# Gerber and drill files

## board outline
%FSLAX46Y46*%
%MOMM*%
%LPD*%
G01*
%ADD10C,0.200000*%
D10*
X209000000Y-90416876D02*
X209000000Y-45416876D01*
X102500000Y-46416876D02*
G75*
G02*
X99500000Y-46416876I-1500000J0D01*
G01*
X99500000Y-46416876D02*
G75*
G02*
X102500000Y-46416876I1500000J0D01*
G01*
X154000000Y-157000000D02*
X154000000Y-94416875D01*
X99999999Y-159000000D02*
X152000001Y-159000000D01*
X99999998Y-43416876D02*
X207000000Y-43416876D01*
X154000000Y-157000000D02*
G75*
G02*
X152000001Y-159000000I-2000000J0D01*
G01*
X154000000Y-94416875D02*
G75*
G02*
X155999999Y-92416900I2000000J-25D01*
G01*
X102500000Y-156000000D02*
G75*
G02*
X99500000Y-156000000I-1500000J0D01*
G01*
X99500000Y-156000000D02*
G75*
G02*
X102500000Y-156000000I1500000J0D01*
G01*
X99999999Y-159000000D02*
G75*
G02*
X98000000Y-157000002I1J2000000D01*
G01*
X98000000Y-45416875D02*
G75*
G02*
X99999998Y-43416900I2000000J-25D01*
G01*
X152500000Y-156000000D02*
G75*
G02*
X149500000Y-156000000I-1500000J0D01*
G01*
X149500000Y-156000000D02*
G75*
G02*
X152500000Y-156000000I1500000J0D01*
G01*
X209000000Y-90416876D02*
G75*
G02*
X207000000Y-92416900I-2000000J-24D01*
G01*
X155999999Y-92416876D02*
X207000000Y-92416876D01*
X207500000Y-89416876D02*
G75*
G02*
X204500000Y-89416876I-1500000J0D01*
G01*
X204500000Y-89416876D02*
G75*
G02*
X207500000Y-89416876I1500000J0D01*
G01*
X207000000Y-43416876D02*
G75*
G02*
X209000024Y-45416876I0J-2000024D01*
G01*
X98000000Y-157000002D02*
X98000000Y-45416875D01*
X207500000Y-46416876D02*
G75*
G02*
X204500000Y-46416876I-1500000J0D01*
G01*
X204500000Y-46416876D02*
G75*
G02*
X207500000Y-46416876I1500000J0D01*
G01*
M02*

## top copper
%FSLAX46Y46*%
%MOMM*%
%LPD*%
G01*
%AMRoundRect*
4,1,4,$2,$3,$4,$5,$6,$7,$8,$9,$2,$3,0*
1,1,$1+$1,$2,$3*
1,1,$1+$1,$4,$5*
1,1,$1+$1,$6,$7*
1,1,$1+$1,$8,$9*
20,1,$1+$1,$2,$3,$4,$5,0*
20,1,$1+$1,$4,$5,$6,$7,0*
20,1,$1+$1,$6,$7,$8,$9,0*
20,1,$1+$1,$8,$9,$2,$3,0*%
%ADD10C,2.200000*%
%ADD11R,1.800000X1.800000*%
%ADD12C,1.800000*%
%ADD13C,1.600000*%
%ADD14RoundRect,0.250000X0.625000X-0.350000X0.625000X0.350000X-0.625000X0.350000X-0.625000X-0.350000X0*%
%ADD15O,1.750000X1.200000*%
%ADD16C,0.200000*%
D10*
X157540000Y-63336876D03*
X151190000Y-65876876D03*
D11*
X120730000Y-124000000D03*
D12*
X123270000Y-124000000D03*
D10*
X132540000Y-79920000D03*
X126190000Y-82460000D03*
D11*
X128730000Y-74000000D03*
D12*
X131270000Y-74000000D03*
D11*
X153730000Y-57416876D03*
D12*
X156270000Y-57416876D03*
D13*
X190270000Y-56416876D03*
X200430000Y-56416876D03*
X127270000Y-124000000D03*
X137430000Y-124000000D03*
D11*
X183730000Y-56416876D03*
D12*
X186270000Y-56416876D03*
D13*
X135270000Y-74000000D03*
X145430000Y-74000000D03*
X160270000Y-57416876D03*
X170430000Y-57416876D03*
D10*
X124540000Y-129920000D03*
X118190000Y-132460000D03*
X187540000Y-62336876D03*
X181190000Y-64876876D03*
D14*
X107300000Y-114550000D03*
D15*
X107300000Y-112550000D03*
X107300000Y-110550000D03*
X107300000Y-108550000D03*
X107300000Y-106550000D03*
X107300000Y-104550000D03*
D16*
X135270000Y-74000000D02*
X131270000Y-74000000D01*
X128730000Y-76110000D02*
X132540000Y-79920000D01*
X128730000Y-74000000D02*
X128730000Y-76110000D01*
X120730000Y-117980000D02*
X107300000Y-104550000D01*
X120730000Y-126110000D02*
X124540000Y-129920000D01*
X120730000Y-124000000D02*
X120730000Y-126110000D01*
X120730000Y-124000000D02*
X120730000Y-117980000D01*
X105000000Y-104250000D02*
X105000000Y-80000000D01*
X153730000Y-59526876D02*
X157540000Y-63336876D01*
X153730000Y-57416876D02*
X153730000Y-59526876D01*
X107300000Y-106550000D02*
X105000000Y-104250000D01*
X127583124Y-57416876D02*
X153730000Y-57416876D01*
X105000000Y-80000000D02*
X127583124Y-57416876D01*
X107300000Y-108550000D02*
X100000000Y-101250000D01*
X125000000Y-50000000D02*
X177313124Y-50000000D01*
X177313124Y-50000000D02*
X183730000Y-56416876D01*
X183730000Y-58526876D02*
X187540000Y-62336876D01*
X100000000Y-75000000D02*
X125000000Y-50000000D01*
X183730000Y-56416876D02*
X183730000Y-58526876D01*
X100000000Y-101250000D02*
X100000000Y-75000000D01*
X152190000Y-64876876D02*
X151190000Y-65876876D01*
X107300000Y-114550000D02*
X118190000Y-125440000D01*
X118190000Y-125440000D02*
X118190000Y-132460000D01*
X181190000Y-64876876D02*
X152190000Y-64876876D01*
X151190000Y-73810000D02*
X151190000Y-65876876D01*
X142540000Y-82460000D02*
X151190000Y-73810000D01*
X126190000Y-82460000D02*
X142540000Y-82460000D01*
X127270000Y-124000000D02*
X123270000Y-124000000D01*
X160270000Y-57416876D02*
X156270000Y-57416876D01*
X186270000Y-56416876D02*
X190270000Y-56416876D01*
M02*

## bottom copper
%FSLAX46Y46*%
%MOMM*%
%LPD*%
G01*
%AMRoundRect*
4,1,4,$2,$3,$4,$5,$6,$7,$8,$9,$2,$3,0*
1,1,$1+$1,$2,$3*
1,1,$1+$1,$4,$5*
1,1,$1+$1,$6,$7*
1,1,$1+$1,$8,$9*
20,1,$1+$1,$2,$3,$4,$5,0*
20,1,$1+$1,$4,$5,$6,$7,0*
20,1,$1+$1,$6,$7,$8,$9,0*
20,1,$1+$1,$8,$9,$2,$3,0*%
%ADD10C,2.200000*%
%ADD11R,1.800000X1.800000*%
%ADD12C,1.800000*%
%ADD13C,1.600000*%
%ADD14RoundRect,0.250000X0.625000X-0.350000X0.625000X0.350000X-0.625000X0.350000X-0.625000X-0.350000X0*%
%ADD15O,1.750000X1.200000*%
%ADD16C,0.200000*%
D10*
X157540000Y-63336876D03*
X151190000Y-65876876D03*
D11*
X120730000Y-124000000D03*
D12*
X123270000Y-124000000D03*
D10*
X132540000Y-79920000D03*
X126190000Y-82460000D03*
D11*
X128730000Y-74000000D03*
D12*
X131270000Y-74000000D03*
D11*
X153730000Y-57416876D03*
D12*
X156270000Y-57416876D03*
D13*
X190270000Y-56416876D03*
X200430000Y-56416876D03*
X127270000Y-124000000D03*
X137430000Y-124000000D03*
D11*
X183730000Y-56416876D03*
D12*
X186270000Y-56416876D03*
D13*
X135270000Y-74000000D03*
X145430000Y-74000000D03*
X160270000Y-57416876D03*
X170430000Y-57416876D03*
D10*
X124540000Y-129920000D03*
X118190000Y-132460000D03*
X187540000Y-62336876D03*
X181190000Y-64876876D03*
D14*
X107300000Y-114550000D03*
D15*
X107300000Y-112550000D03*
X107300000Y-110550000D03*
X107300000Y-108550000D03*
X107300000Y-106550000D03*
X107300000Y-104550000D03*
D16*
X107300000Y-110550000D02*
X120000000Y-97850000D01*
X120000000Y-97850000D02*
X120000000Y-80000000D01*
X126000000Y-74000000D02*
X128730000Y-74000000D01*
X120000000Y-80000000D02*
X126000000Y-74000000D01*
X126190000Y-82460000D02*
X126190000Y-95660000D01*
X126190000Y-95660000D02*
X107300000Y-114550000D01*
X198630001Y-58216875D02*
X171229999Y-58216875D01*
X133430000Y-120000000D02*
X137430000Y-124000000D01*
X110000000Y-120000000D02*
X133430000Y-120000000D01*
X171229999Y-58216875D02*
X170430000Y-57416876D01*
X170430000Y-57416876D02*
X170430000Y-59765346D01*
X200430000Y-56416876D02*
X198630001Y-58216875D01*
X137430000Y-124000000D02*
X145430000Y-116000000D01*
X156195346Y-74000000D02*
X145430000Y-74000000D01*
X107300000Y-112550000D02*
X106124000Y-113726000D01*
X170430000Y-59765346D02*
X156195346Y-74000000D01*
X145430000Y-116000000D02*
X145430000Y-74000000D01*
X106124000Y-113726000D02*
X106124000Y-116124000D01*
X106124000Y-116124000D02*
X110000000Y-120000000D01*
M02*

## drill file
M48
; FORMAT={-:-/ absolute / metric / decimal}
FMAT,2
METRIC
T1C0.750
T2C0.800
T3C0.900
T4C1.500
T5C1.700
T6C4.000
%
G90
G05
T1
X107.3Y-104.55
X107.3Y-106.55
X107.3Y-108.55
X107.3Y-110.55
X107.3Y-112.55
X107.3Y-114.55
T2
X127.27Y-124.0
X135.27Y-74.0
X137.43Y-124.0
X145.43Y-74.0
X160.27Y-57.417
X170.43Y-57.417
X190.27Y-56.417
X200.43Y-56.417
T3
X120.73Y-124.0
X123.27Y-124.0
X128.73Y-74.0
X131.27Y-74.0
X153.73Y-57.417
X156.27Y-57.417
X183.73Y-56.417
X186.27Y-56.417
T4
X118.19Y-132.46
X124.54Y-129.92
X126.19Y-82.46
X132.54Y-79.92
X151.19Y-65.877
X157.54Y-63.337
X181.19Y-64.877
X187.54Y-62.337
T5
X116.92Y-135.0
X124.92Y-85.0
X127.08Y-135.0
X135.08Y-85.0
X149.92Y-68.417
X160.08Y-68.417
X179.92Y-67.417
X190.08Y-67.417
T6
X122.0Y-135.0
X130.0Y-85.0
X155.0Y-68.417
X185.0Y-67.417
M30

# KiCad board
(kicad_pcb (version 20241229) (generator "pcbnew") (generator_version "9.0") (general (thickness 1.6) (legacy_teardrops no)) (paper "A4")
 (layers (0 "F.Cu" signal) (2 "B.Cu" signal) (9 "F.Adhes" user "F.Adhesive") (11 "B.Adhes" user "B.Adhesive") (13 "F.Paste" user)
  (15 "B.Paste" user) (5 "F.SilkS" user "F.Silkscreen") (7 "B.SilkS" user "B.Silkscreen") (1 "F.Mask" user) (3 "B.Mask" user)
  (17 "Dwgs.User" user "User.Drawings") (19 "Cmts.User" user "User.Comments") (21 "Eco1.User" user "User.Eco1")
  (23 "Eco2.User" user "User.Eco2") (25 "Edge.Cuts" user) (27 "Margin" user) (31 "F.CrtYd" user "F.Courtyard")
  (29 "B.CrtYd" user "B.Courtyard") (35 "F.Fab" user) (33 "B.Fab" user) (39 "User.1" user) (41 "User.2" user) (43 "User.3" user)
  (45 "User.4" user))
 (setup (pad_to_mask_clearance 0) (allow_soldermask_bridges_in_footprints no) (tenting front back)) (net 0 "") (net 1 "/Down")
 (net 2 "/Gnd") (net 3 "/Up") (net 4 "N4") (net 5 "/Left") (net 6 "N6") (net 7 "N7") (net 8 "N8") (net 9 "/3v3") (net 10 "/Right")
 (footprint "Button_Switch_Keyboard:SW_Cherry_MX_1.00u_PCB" (layer "F.Cu") (at 157.54 63.336876)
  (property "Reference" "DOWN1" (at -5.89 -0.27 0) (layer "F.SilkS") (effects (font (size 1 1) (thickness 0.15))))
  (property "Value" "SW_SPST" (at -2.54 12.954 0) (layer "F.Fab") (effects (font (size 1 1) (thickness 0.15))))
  (pad "" np_thru_hole circle (at -7.62 5.08) (size 1.7 1.7) (drill 1.7) (layers "*.Cu" "*.Mask"))
  (pad "" np_thru_hole circle (at -2.54 5.08) (size 4 4) (drill 4) (layers "*.Cu" "*.Mask"))
  (pad "" np_thru_hole circle (at 2.54 5.08) (size 1.7 1.7) (drill 1.7) (layers "*.Cu" "*.Mask"))
  (pad "1" thru_hole circle (at 0 0) (size 2.2 2.2) (drill 1.5) (layers "*.Cu" "*.Mask") (remove_unused_layers no) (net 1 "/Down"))
  (pad "2" thru_hole circle (at -6.35 2.54) (size 2.2 2.2) (drill 1.5) (layers "*.Cu" "*.Mask") (remove_unused_layers no) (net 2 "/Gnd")))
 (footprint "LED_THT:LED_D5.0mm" (layer "F.Cu") (at 120.73 124)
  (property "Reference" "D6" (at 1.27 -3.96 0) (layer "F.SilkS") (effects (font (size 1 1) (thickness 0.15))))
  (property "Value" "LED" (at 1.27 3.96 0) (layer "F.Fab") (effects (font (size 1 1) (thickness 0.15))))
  (pad "1" thru_hole rect (at 0 0) (size 1.8 1.8) (drill 0.9) (layers "*.Cu" "*.Mask") (remove_unused_layers no) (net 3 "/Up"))
  (pad "2" thru_hole circle (at 2.54 0) (size 1.8 1.8) (drill 0.9) (layers "*.Cu" "*.Mask") (remove_unused_layers no) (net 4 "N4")))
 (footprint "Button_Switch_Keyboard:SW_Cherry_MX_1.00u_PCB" (layer "F.Cu") (at 132.54 79.92)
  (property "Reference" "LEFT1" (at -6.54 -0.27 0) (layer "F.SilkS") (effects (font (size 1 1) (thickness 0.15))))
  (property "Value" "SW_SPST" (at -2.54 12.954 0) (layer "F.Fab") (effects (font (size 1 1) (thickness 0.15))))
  (pad "" np_thru_hole circle (at -7.62 5.08) (size 1.7 1.7) (drill 1.7) (layers "*.Cu" "*.Mask"))
  (pad "" np_thru_hole circle (at -2.54 5.08) (size 4 4) (drill 4) (layers "*.Cu" "*.Mask"))
  (pad "" np_thru_hole circle (at 2.54 5.08) (size 1.7 1.7) (drill 1.7) (layers "*.Cu" "*.Mask"))
  (pad "1" thru_hole circle (at 0 0) (size 2.2 2.2) (drill 1.5) (layers "*.Cu" "*.Mask") (remove_unused_layers no) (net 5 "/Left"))
  (pad "2" thru_hole circle (at -6.35 2.54) (size 2.2 2.2) (drill 1.5) (layers "*.Cu" "*.Mask") (remove_unused_layers no) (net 2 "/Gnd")))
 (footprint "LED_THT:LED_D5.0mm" (layer "F.Cu") (at 128.73 74)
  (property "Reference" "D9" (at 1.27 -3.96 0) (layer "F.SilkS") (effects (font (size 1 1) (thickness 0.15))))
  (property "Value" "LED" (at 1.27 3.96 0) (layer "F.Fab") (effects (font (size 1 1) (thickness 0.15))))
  (pad "1" thru_hole rect (at 0 0) (size 1.8 1.8) (drill 0.9) (layers "*.Cu" "*.Mask") (remove_unused_layers no) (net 5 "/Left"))
  (pad "2" thru_hole circle (at 2.54 0) (size 1.8 1.8) (drill 0.9) (layers "*.Cu" "*.Mask") (remove_unused_layers no) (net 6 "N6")))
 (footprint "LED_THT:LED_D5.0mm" (layer "F.Cu") (at 153.73 57.416876)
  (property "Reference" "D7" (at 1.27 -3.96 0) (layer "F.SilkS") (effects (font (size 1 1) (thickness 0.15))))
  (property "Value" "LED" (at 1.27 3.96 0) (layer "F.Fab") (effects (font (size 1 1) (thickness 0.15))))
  (pad "1" thru_hole rect (at 0 0) (size 1.8 1.8) (drill 0.9) (layers "*.Cu" "*.Mask") (remove_unused_layers no) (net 1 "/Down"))
  (pad "2" thru_hole circle (at 2.54 0) (size 1.8 1.8) (drill 0.9) (layers "*.Cu" "*.Mask") (remove_unused_layers no) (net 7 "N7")))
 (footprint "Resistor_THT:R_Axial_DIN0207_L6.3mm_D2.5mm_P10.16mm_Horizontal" (layer "F.Cu") (at 190.27 56.416876)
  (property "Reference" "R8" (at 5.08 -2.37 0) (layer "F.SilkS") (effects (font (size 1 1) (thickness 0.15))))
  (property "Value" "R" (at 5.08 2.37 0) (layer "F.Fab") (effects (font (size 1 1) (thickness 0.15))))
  (pad "1" thru_hole circle (at 0 0) (size 1.6 1.6) (drill 0.8) (layers "*.Cu" "*.Mask") (remove_unused_layers no) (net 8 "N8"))
  (pad "2" thru_hole circle (at 10.16 0) (size 1.6 1.6) (drill 0.8) (layers "*.Cu" "*.Mask") (remove_unused_layers no) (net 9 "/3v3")))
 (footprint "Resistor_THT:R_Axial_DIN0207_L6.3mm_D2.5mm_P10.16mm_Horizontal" (layer "F.Cu") (at 127.27 124)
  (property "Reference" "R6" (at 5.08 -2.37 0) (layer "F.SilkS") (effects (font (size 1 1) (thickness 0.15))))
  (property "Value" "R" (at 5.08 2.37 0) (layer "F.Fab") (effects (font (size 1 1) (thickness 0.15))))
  (pad "1" thru_hole circle (at 0 0) (size 1.6 1.6) (drill 0.8) (layers "*.Cu" "*.Mask") (remove_unused_layers no) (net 4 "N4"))
  (pad "2" thru_hole circle (at 10.16 0) (size 1.6 1.6) (drill 0.8) (layers "*.Cu" "*.Mask") (remove_unused_layers no) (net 9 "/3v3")))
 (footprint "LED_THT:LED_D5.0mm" (layer "F.Cu") (at 183.73 56.416876)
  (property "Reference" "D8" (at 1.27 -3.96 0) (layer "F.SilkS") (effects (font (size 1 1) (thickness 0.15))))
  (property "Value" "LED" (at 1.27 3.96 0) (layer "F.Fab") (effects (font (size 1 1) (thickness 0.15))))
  (pad "1" thru_hole rect (at 0 0) (size 1.8 1.8) (drill 0.9) (layers "*.Cu" "*.Mask") (remove_unused_layers no) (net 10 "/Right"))
  (pad "2" thru_hole circle (at 2.54 0) (size 1.8 1.8) (drill 0.9) (layers "*.Cu" "*.Mask") (remove_unused_layers no) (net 8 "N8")))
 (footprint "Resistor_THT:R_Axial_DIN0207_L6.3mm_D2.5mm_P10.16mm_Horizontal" (layer "F.Cu") (at 135.27 74)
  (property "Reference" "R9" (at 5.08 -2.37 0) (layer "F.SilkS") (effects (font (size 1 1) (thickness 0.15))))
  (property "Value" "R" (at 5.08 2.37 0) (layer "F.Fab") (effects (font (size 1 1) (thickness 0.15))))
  (pad "1" thru_hole circle (at 0 0) (size 1.6 1.6) (drill 0.8) (layers "*.Cu" "*.Mask") (remove_unused_layers no) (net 6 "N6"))
  (pad "2" thru_hole circle (at 10.16 0) (size 1.6 1.6) (drill 0.8) (layers "*.Cu" "*.Mask") (remove_unused_layers no) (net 9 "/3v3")))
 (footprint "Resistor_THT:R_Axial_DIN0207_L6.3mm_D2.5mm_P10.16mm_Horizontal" (layer "F.Cu") (at 160.27 57.416876)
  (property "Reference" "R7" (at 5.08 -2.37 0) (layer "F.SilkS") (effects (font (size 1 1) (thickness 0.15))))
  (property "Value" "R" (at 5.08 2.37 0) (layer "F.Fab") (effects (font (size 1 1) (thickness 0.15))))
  (pad "1" thru_hole circle (at 0 0) (size 1.6 1.6) (drill 0.8) (layers "*.Cu" "*.Mask") (remove_unused_layers no) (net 7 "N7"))
  (pad "2" thru_hole circle (at 10.16 0) (size 1.6 1.6) (drill 0.8) (layers "*.Cu" "*.Mask") (remove_unused_layers no) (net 9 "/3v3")))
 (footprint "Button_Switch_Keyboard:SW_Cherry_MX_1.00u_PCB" (layer "F.Cu") (at 124.54 129.92)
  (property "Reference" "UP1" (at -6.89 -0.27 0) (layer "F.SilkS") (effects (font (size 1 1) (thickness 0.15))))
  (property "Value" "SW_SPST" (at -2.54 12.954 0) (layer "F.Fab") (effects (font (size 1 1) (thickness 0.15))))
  (pad "" np_thru_hole circle (at -7.62 5.08) (size 1.7 1.7) (drill 1.7) (layers "*.Cu" "*.Mask"))
  (pad "" np_thru_hole circle (at -2.54 5.08) (size 4 4) (drill 4) (layers "*.Cu" "*.Mask"))
  (pad "" np_thru_hole circle (at 2.54 5.08) (size 1.7 1.7) (drill 1.7) (layers "*.Cu" "*.Mask"))
  (pad "1" thru_hole circle (at 0 0) (size 2.2 2.2) (drill 1.5) (layers "*.Cu" "*.Mask") (remove_unused_layers no) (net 3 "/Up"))
  (pad "2" thru_hole circle (at -6.35 2.54) (size 2.2 2.2) (drill 1.5) (layers "*.Cu" "*.Mask") (remove_unused_layers no) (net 2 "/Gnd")))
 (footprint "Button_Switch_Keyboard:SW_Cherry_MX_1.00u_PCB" (layer "F.Cu") (at 187.54 62.336876)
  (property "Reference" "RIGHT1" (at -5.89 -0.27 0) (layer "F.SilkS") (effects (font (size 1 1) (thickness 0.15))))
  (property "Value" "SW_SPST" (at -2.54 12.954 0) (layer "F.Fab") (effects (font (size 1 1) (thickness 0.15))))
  (pad "" np_thru_hole circle (at -7.62 5.08) (size 1.7 1.7) (drill 1.7) (layers "*.Cu" "*.Mask"))
  (pad "" np_thru_hole circle (at -2.54 5.08) (size 4 4) (drill 4) (layers "*.Cu" "*.Mask"))
  (pad "" np_thru_hole circle (at 2.54 5.08) (size 1.7 1.7) (drill 1.7) (layers "*.Cu" "*.Mask"))
  (pad "1" thru_hole circle (at 0 0) (size 2.2 2.2) (drill 1.5) (layers "*.Cu" "*.Mask") (remove_unused_layers no) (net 10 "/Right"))
  (pad "2" thru_hole circle (at -6.35 2.54) (size 2.2 2.2) (drill 1.5) (layers "*.Cu" "*.Mask") (remove_unused_layers no) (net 2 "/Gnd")))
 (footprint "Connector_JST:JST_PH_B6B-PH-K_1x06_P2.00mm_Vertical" (layer "B.Cu") (at 107.3 114.55 90)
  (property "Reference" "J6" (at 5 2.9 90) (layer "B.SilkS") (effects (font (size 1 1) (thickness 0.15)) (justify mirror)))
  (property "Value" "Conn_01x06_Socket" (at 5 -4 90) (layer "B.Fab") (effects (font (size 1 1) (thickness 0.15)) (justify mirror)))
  (pad "1" thru_hole roundrect (at 0 0 90) (size 1.2 1.75) (drill 0.75) (layers "*.Cu" "*.Mask") (remove_unused_layers no)
   (roundrect_rratio 0.208333) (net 2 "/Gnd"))
  (pad "2" thru_hole oval (at 2 0 90) (size 1.2 1.75) (drill 0.75) (layers "*.Cu" "*.Mask") (remove_unused_layers no) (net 9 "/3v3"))
  (pad "3" thru_hole oval (at 4 0 90) (size 1.2 1.75) (drill 0.75) (layers "*.Cu" "*.Mask") (remove_unused_layers no) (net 5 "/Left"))
  (pad "4" thru_hole oval (at 6 0 90) (size 1.2 1.75) (drill 0.75) (layers "*.Cu" "*.Mask") (remove_unused_layers no) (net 10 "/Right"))
  (pad "5" thru_hole oval (at 8 0 90) (size 1.2 1.75) (drill 0.75) (layers "*.Cu" "*.Mask") (remove_unused_layers no) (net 1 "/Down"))
  (pad "6" thru_hole oval (at 10 0 90) (size 1.2 1.75) (drill 0.75) (layers "*.Cu" "*.Mask") (remove_unused_layers no) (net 3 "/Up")))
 (gr_line (start 209 90.416876) (end 209 45.416876) (stroke (width 0.2) (type default)) (layer "Edge.Cuts"))
 (gr_circle (center 101 46.416876) (end 102.5 46.416876) (stroke (width 0.2) (type default)) (fill no) (layer "Edge.Cuts"))
 (gr_line (start 154 157) (end 154 94.416875) (stroke (width 0.2) (type default)) (layer "Edge.Cuts"))
 (gr_line (start 99.999999 159) (end 152.000001 159) (stroke (width 0.2) (type default)) (layer "Edge.Cuts"))
 (gr_line (start 99.999998 43.416876) (end 207 43.416876) (stroke (width 0.2) (type default)) (layer "Edge.Cuts"))
 (gr_arc (start 154 157) (mid 153.414214 158.414214) (end 152.000001 159) (stroke (width 0.2) (type default)) (layer "Edge.Cuts"))
 (gr_arc (start 154 94.416875) (mid 154.585786 93.002662) (end 155.999999 92.416876) (stroke (width 0.2) (type default)) (layer "Edge.Cuts"))
 (gr_circle (center 101 156) (end 102.5 156) (stroke (width 0.2) (type default)) (fill no) (layer "Edge.Cuts"))
 (gr_arc (start 99.999999 159) (mid 98.585786 158.414214) (end 98 157.000002) (stroke (width 0.2) (type default)) (layer "Edge.Cuts"))
 (gr_arc (start 98 45.416875) (mid 98.585786 44.002662) (end 99.999998 43.416876) (stroke (width 0.2) (type default)) (layer "Edge.Cuts"))
 (gr_circle (center 151 156) (end 152.5 156) (stroke (width 0.2) (type default)) (fill no) (layer "Edge.Cuts"))
 (gr_arc (start 209 90.416876) (mid 208.414214 91.83109) (end 207 92.416876) (stroke (width 0.2) (type default)) (layer "Edge.Cuts"))
 (gr_line (start 155.999999 92.416876) (end 207 92.416876) (stroke (width 0.2) (type default)) (layer "Edge.Cuts"))
 (gr_circle (center 206 89.416876) (end 207.5 89.416876) (stroke (width 0.2) (type default)) (fill no) (layer "Edge.Cuts"))
 (gr_arc (start 207 43.416876) (mid 208.414214 44.002662) (end 209 45.416876) (stroke (width 0.2) (type default)) (layer "Edge.Cuts"))
 (gr_line (start 98 157.000002) (end 98 45.416875) (stroke (width 0.2) (type default)) (layer "Edge.Cuts"))
 (gr_circle (center 206 46.416876) (end 207.5 46.416876) (stroke (width 0.2) (type default)) (fill no) (layer "Edge.Cuts"))
 (segment (start 135.27 74) (end 131.27 74) (width 0.2) (layer "F.Cu") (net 6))
 (segment (start 128.73 76.11) (end 132.54 79.92) (width 0.2) (layer "F.Cu") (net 5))
 (segment (start 128.73 74) (end 128.73 76.11) (width 0.2) (layer "F.Cu") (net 5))
 (segment (start 107.3 110.55) (end 120 97.85) (width 0.2) (layer "B.Cu") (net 5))
 (segment (start 120 97.85) (end 120 80) (width 0.2) (layer "B.Cu") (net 5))
 (segment (start 126 74) (end 128.73 74) (width 0.2) (layer "B.Cu") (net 5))
 (segment (start 120 80) (end 126 74) (width 0.2) (layer "B.Cu") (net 5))
 (segment (start 120.73 117.98) (end 107.3 104.55) (width 0.2) (layer "F.Cu") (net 3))
 (segment (start 120.73 126.11) (end 124.54 129.92) (width 0.2) (layer "F.Cu") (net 3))
 (segment (start 120.73 124) (end 120.73 126.11) (width 0.2) (layer "F.Cu") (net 3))
 (segment (start 120.73 124) (end 120.73 117.98) (width 0.2) (layer "F.Cu") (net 3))
 (segment (start 105 104.25) (end 105 80) (width 0.2) (layer "F.Cu") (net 1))
 (segment (start 153.73 59.526876) (end 157.54 63.336876) (width 0.2) (layer "F.Cu") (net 1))
 (segment (start 153.73 57.416876) (end 153.73 59.526876) (width 0.2) (layer "F.Cu") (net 1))
 (segment (start 107.3 106.55) (end 105 104.25) (width 0.2) (layer "F.Cu") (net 1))
 (segment (start 127.583124 57.416876) (end 153.73 57.416876) (width 0.2) (layer "F.Cu") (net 1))
 (segment (start 105 80) (end 127.583124 57.416876) (width 0.2) (layer "F.Cu") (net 1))
 (segment (start 107.3 108.55) (end 100 101.25) (width 0.2) (layer "F.Cu") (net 10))
 (segment (start 125 50) (end 177.313124 50) (width 0.2) (layer "F.Cu") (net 10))
 (segment (start 177.313124 50) (end 183.73 56.416876) (width 0.2) (layer "F.Cu") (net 10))
 (segment (start 183.73 58.526876) (end 187.54 62.336876) (width 0.2) (layer "F.Cu") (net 10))
 (segment (start 100 75) (end 125 50) (width 0.2) (layer "F.Cu") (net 10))
 (segment (start 183.73 56.416876) (end 183.73 58.526876) (width 0.2) (layer "F.Cu") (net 10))
 (segment (start 100 101.25) (end 100 75) (width 0.2) (layer "F.Cu") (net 10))
 (segment (start 152.19 64.876876) (end 151.19 65.876876) (width 0.2) (layer "F.Cu") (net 2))
 (segment (start 107.3 114.55) (end 118.19 125.44) (width 0.2) (layer "F.Cu") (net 2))
 (segment (start 118.19 125.44) (end 118.19 132.46) (width 0.2) (layer "F.Cu") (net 2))
 (segment (start 181.19 64.876876) (end 152.19 64.876876) (width 0.2) (layer "F.Cu") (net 2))
 (segment (start 151.19 73.81) (end 151.19 65.876876) (width 0.2) (layer "F.Cu") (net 2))
 (segment (start 142.54 82.46) (end 151.19 73.81) (width 0.2) (layer "F.Cu") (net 2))
 (segment (start 126.19 82.46) (end 142.54 82.46) (width 0.2) (layer "F.Cu") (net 2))
 (segment (start 126.19 82.46) (end 126.19 95.66) (width 0.2) (layer "B.Cu") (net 2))
 (segment (start 126.19 95.66) (end 107.3 114.55) (width 0.2) (layer "B.Cu") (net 2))
 (segment (start 198.630001 58.216875) (end 171.229999 58.216875) (width 0.2) (layer "B.Cu") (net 9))
 (segment (start 133.43 120) (end 137.43 124) (width 0.2) (layer "B.Cu") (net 9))
 (segment (start 110 120) (end 133.43 120) (width 0.2) (layer "B.Cu") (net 9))
 (segment (start 171.229999 58.216875) (end 170.43 57.416876) (width 0.2) (layer "B.Cu") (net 9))
 (segment (start 170.43 57.416876) (end 170.43 59.765346) (width 0.2) (layer "B.Cu") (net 9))
 (segment (start 200.43 56.416876) (end 198.630001 58.216875) (width 0.2) (layer "B.Cu") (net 9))
 (segment (start 137.43 124) (end 145.43 116) (width 0.2) (layer "B.Cu") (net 9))
 (segment (start 156.195346 74) (end 145.43 74) (width 0.2) (layer "B.Cu") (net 9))
 (segment (start 107.3 112.55) (end 106.124 113.726) (width 0.2) (layer "B.Cu") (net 9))
 (segment (start 170.43 59.765346) (end 156.195346 74) (width 0.2) (layer "B.Cu") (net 9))
 (segment (start 145.43 116) (end 145.43 74) (width 0.2) (layer "B.Cu") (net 9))
 (segment (start 106.124 113.726) (end 106.124 116.124) (width 0.2) (layer "B.Cu") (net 9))
 (segment (start 106.124 116.124) (end 110 120) (width 0.2) (layer "B.Cu") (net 9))
 (segment (start 127.27 124) (end 123.27 124) (width 0.2) (layer "F.Cu") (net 4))
 (segment (start 160.27 57.416876) (end 156.27 57.416876) (width 0.2) (layer "F.Cu") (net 7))
 (segment (start 186.27 56.416876) (end 190.27 56.416876) (width 0.2) (layer "F.Cu") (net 8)))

